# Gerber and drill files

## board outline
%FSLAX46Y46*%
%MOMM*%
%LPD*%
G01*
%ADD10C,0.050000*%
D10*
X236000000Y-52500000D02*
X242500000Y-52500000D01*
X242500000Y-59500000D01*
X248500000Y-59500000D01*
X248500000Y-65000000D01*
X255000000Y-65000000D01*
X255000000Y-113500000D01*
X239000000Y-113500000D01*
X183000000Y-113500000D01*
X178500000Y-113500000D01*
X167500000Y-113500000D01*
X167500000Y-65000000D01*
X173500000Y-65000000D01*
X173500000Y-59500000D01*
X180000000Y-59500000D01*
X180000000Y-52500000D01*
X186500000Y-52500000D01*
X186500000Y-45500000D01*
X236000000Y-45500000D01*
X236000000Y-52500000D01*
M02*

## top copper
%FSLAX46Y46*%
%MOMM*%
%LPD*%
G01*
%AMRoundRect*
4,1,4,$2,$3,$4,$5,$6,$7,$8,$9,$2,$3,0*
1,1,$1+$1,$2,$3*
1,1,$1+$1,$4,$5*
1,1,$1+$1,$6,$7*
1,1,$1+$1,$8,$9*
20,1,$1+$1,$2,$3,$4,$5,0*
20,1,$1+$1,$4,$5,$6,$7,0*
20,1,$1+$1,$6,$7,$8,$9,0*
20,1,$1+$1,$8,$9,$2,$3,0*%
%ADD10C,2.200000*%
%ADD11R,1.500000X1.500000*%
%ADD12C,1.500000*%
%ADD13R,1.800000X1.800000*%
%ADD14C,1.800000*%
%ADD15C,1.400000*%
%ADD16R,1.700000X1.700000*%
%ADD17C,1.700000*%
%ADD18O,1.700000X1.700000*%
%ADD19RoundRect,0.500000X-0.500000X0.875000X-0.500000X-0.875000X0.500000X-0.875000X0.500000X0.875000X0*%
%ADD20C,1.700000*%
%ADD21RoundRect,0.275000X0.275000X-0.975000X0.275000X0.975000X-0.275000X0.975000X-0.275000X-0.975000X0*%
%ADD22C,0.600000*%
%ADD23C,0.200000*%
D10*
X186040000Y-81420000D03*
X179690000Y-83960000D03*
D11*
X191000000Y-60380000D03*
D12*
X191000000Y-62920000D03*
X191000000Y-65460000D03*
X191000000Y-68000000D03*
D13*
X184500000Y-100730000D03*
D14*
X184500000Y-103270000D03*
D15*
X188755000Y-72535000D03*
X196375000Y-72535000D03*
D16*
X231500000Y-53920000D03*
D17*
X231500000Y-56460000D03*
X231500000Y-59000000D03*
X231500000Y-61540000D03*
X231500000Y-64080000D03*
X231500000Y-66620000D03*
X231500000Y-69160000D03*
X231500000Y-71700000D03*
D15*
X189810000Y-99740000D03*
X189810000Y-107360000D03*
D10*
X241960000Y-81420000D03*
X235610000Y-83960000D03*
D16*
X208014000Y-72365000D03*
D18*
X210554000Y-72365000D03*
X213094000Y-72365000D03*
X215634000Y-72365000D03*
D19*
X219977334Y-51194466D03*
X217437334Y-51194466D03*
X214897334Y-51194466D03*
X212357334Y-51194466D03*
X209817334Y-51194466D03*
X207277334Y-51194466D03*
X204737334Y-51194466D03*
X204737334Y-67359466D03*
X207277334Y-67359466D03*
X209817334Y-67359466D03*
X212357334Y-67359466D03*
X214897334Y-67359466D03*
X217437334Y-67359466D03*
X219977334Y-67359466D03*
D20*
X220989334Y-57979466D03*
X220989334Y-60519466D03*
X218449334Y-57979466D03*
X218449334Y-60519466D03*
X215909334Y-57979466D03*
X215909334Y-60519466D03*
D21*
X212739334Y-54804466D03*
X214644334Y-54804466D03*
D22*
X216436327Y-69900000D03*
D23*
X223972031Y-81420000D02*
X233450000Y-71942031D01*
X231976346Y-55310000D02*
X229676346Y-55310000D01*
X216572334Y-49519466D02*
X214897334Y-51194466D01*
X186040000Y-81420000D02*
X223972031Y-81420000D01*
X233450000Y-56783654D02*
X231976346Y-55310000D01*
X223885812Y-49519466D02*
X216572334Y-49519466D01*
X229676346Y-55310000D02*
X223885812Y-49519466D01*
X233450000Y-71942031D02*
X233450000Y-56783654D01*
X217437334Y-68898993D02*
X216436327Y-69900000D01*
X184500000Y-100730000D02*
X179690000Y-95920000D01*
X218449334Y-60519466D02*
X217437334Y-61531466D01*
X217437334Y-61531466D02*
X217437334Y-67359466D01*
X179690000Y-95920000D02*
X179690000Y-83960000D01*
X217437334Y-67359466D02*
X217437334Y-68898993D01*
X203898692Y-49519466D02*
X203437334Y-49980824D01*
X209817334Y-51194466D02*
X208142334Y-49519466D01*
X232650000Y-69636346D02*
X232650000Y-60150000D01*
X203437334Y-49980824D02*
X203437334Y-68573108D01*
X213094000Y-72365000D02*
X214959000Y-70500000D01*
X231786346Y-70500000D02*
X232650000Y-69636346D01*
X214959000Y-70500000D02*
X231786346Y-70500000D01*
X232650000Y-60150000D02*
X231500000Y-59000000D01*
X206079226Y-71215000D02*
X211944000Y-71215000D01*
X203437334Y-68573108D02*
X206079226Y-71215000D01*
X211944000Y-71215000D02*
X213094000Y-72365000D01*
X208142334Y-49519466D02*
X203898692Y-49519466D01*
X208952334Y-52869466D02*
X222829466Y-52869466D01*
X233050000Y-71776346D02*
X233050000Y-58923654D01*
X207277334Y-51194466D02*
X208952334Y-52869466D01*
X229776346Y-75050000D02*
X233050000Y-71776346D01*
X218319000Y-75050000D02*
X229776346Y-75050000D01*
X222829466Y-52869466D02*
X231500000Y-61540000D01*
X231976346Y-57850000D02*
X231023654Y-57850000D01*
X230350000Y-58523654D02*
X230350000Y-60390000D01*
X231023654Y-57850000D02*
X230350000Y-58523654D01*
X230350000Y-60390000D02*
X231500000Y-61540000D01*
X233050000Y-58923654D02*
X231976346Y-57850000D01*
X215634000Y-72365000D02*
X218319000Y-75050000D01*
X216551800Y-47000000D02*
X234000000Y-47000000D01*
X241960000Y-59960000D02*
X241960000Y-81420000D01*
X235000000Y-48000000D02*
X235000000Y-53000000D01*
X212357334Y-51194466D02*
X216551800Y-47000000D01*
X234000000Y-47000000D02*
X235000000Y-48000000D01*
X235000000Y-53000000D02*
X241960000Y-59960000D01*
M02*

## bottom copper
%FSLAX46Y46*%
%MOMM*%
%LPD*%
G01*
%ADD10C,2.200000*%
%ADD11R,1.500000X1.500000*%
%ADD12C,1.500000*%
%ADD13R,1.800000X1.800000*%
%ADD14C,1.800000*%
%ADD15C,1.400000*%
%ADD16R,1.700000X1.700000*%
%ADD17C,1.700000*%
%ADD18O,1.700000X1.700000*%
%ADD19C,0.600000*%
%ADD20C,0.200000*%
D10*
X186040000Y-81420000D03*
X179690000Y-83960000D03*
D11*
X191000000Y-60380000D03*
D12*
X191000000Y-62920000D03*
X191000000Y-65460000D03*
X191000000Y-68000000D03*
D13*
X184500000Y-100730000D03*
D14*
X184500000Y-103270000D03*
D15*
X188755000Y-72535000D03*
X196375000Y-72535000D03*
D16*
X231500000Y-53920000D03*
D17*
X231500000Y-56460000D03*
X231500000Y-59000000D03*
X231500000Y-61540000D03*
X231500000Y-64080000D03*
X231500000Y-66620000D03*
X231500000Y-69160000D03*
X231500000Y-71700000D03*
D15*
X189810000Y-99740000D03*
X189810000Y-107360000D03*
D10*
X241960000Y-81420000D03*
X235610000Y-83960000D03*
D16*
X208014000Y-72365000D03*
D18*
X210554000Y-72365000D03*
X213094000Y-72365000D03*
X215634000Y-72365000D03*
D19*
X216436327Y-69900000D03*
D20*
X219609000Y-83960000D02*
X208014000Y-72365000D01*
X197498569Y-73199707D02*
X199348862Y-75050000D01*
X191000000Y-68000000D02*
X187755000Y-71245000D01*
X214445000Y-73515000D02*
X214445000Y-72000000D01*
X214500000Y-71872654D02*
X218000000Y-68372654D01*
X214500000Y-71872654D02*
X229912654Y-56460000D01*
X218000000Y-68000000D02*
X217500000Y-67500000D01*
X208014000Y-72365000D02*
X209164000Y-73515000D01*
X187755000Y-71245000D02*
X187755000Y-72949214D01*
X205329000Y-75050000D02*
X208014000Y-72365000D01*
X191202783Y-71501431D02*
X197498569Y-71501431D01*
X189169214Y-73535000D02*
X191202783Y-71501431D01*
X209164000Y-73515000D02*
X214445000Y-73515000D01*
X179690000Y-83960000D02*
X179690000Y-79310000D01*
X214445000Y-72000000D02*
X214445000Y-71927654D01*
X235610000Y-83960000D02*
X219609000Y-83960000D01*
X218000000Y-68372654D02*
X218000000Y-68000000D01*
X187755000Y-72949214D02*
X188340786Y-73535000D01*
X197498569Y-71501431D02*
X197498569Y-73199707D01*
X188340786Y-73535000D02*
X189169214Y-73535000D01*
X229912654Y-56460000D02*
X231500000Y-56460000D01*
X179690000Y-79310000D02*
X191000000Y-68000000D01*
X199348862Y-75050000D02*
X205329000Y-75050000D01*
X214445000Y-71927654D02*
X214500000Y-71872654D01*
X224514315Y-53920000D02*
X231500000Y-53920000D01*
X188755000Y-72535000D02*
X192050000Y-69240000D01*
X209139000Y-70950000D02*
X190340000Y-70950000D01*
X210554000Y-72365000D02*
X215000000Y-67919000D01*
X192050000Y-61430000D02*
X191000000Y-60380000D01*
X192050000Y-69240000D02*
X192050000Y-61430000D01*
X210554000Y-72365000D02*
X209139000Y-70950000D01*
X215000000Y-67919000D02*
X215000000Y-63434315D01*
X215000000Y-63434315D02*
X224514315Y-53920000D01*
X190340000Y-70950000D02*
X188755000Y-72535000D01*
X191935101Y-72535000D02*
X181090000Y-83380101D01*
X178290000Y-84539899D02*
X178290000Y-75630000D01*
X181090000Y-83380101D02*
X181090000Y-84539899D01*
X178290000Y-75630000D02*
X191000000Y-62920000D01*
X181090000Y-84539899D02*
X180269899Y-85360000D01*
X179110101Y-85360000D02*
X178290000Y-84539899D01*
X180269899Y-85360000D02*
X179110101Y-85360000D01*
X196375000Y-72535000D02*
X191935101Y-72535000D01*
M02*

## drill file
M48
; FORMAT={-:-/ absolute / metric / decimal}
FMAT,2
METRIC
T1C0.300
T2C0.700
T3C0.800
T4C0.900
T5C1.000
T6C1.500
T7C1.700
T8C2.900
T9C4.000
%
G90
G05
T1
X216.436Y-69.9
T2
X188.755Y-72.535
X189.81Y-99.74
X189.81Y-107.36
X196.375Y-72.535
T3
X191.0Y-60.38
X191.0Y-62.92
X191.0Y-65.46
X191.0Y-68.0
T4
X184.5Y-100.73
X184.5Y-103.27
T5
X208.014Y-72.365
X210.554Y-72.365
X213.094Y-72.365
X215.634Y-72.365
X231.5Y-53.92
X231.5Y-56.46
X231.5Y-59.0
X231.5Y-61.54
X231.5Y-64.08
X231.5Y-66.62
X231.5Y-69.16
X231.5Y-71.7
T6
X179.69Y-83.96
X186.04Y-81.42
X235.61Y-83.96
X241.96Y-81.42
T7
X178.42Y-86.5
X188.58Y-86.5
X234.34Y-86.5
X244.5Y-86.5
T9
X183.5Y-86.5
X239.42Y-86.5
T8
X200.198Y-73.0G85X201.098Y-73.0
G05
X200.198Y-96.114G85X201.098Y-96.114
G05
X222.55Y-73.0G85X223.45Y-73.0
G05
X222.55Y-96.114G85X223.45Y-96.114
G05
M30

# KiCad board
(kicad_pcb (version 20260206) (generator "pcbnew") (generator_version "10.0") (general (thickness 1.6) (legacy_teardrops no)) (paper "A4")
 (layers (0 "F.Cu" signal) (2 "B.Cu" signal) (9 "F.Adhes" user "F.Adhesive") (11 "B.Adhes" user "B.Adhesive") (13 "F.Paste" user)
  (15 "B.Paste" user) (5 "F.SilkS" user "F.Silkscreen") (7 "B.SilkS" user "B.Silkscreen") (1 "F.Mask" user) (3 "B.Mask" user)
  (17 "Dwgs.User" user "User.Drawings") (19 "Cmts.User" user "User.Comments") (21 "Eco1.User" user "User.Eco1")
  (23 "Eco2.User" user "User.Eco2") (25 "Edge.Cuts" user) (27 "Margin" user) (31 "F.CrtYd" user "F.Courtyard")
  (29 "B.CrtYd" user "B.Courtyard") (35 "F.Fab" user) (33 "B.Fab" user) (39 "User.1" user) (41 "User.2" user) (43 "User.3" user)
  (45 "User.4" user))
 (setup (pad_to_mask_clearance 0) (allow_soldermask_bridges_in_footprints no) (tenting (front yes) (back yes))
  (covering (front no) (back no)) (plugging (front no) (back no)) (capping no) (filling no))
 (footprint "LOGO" (layer "F.Cu") (at 224.5 107)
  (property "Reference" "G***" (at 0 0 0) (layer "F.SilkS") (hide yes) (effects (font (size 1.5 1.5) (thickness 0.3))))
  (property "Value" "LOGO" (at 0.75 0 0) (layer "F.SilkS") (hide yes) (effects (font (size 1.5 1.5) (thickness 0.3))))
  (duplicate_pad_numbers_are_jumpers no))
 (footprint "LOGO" (layer "F.Cu") (at 238 54)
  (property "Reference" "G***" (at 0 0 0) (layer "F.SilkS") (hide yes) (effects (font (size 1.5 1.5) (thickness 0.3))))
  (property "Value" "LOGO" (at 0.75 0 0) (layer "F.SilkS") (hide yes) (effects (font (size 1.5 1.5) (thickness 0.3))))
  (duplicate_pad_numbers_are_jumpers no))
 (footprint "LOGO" (layer "F.Cu") (at 202.605439 106.48253)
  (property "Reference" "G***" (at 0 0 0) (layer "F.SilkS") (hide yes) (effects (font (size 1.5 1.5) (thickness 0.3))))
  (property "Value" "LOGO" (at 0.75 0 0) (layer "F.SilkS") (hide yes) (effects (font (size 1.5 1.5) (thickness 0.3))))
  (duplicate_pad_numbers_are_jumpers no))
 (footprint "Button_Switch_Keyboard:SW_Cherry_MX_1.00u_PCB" (layer "F.Cu") (at 186.04 81.42)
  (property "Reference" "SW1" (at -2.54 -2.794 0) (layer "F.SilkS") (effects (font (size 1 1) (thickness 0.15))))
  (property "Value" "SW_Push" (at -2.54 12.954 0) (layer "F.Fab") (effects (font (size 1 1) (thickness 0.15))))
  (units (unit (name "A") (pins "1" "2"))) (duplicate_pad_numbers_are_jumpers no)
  (pad "" np_thru_hole circle (at -7.62 5.08) (size 1.7 1.7) (drill 1.7) (layers "*.Cu" "*.Mask"))
  (pad "" np_thru_hole circle (at -2.54 5.08) (size 4 4) (drill 4) (layers "*.Cu" "*.Mask"))
  (pad "" np_thru_hole circle (at 2.54 5.08) (size 1.7 1.7) (drill 1.7) (layers "*.Cu" "*.Mask"))
  (pad "1" thru_hole circle (at 0 0) (size 2.2 2.2) (drill 1.5) (layers "*.Cu" "*.Mask") (remove_unused_layers no) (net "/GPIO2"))
  (pad "2" thru_hole circle (at -6.35 2.54) (size 2.2 2.2) (drill 1.5) (layers "*.Cu" "*.Mask") (remove_unused_layers no) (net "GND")))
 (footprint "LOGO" (layer "F.Cu") (at 172.5 71.5)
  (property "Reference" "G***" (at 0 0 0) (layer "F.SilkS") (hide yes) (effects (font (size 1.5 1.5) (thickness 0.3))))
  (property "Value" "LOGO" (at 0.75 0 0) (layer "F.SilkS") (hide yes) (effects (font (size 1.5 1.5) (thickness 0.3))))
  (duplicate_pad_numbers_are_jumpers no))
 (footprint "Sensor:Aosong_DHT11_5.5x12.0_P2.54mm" (layer "F.Cu") (at 191 60.38)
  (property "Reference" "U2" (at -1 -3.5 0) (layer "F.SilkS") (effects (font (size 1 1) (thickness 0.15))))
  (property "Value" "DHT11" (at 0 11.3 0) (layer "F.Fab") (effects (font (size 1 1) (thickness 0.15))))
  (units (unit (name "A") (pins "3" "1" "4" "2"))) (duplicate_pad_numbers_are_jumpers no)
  (pad "1" thru_hole rect (at 0 0) (size 1.5 1.5) (drill 0.8) (layers "*.Cu" "*.Mask") (remove_unused_layers no) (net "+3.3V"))
  (pad "2" thru_hole circle (at 0 2.54) (size 1.5 1.5) (drill 0.8) (layers "*.Cu" "*.Mask") (remove_unused_layers no) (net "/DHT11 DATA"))
  (pad "3" thru_hole circle (at 0 5.08) (size 1.5 1.5) (drill 0.8) (layers "*.Cu" "*.Mask") (remove_unused_layers no)
   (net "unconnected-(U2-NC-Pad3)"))
  (pad "4" thru_hole circle (at 0 7.62) (size 1.5 1.5) (drill 0.8) (layers "*.Cu" "*.Mask") (remove_unused_layers no) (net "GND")))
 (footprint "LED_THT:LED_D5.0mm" (layer "F.Cu") (at 184.5 100.73 -90)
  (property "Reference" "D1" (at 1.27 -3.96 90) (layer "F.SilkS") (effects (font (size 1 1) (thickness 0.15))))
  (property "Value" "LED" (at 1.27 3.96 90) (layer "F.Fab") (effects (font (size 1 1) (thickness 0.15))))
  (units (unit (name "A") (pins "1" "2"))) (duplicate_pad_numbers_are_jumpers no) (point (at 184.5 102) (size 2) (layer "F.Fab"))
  (pad "1" thru_hole rect (at 0 0 270) (size 1.8 1.8) (drill 0.9) (layers "*.Cu" "*.Mask") (remove_unused_layers no) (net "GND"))
  (pad "2" thru_hole circle (at 2.54 0 270) (size 1.8 1.8) (drill 0.9) (layers "*.Cu" "*.Mask") (remove_unused_layers no)))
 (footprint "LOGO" (layer "F.Cu") (at 248.5 70)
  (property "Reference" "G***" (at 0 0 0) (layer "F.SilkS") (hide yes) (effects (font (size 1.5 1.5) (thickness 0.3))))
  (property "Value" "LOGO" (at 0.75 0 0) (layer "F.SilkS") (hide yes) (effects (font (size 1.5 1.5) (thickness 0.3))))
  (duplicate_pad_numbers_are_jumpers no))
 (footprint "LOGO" (layer "F.Cu") (at 194 51)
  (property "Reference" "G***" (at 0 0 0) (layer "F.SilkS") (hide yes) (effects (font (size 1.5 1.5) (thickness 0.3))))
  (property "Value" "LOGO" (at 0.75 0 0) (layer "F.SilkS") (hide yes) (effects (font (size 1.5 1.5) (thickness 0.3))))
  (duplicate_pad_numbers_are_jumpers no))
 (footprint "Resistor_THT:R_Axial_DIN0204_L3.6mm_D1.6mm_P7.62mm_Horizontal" (layer "F.Cu") (at 188.755 72.535)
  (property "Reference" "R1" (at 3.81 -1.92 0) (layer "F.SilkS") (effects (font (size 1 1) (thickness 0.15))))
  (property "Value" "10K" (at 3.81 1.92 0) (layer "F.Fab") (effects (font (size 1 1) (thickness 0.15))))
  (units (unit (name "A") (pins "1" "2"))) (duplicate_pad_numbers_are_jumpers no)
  (pad "1" thru_hole circle (at 0 0) (size 1.4 1.4) (drill 0.7) (layers "*.Cu" "*.Mask") (remove_unused_layers no) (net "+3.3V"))
  (pad "2" thru_hole circle (at 7.62 0) (size 1.4 1.4) (drill 0.7) (layers "*.Cu" "*.Mask") (remove_unused_layers no) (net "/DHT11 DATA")))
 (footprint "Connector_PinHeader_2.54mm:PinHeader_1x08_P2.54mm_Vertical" (layer "F.Cu") (at 231.5 53.92)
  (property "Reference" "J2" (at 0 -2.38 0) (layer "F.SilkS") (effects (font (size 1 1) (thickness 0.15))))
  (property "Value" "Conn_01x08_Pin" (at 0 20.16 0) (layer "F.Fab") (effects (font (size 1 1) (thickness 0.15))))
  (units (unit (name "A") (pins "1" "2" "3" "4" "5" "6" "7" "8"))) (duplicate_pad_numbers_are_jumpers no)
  (pad "1" thru_hole rect (at 0 0) (size 1.7 1.7) (drill 1) (layers "*.Cu" "*.Mask") (remove_unused_layers no) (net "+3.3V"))
  (pad "2" thru_hole circle (at 0 2.54) (size 1.7 1.7) (drill 1) (layers "*.Cu" "*.Mask") (remove_unused_layers no) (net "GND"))
  (pad "3" thru_hole circle (at 0 5.08) (size 1.7 1.7) (drill 1) (layers "*.Cu" "*.Mask") (remove_unused_layers no) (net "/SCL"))
  (pad "4" thru_hole circle (at 0 7.62) (size 1.7 1.7) (drill 1) (layers "*.Cu" "*.Mask") (remove_unused_layers no) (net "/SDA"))
  (pad "5" thru_hole circle (at 0 10.16) (size 1.7 1.7) (drill 1) (layers "*.Cu" "*.Mask") (remove_unused_layers no)
   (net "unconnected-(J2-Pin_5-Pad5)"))
  (pad "6" thru_hole circle (at 0 12.7) (size 1.7 1.7) (drill 1) (layers "*.Cu" "*.Mask") (remove_unused_layers no)
   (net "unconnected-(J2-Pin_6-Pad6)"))
  (pad "7" thru_hole circle (at 0 15.24) (size 1.7 1.7) (drill 1) (layers "*.Cu" "*.Mask") (remove_unused_layers no)
   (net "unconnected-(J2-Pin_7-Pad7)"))
  (pad "8" thru_hole circle (at 0 17.78) (size 1.7 1.7) (drill 1) (layers "*.Cu" "*.Mask") (remove_unused_layers no)
   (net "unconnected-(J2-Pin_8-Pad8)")))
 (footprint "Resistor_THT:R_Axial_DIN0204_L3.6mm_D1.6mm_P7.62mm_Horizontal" (layer "F.Cu") (at 189.81 99.74 -90)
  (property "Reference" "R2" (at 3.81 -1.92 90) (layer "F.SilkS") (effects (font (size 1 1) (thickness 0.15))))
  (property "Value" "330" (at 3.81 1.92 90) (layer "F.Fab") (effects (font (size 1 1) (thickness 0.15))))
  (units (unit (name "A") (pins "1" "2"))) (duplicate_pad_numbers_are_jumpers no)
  (pad "1" thru_hole circle (at 0 0 270) (size 1.4 1.4) (drill 0.7) (layers "*.Cu" "*.Mask") (remove_unused_layers no) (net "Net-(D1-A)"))
  (pad "2" thru_hole circle (at 7.62 0 270) (size 1.4 1.4) (drill 0.7) (layers "*.Cu" "*.Mask") (remove_unused_layers no)))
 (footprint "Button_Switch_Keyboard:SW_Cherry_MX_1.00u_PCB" (layer "F.Cu") (at 241.96 81.42)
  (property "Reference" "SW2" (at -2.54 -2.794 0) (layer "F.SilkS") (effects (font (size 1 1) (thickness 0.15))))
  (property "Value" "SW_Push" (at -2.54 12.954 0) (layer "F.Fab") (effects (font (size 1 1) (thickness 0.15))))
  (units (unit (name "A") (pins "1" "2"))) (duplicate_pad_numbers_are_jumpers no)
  (pad "" np_thru_hole circle (at -7.62 5.08) (size 1.7 1.7) (drill 1.7) (layers "*.Cu" "*.Mask"))
  (pad "" np_thru_hole circle (at -2.54 5.08) (size 4 4) (drill 4) (layers "*.Cu" "*.Mask"))
  (pad "" np_thru_hole circle (at 2.54 5.08) (size 1.7 1.7) (drill 1.7) (layers "*.Cu" "*.Mask"))
  (pad "1" thru_hole circle (at 0 0) (size 2.2 2.2) (drill 1.5) (layers "*.Cu" "*.Mask") (remove_unused_layers no) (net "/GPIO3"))
  (pad "2" thru_hole circle (at -6.35 2.54) (size 2.2 2.2) (drill 1.5) (layers "*.Cu" "*.Mask") (remove_unused_layers no) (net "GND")))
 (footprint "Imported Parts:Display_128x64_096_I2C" (layer "F.Cu") (at 211.824 72.365)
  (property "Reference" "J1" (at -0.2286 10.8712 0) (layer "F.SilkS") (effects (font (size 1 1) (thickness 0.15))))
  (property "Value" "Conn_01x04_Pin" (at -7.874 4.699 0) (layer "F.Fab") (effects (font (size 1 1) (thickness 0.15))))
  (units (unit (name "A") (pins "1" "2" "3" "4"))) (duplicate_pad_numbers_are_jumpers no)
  (pad "" np_thru_hole oval (at -11.176 0.635) (size 3.8 2.9) (drill oval 3.8 2.9) (layers "*.Cu" "*.Mask"))
  (pad "" np_thru_hole oval (at -11.176 23.749) (size 3.8 2.9) (drill oval 3.8 2.9) (layers "*.Cu" "*.Mask"))
  (pad "" np_thru_hole oval (at 11.176 0.635) (size 3.8 2.9) (drill oval 3.8 2.9) (layers "*.Cu" "*.Mask"))
  (pad "" np_thru_hole oval (at 11.176 23.749) (size 3.8 2.9) (drill oval 3.8 2.9) (layers "*.Cu" "*.Mask"))
  (pad "1" thru_hole rect (at -3.81 0 90) (size 1.7 1.7) (drill 1) (layers "*.Cu" "*.Mask") (remove_unused_layers no) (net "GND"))
  (pad "2" thru_hole oval (at -1.27 0 90) (size 1.7 1.7) (drill 1) (layers "*.Cu" "*.Mask") (remove_unused_layers no) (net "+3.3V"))
  (pad "3" thru_hole oval (at 1.27 0 90) (size 1.7 1.7) (drill 1) (layers "*.Cu" "*.Mask") (remove_unused_layers no) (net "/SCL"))
  (pad "4" thru_hole oval (at 3.81 0 90) (size 1.7 1.7) (drill 1) (layers "*.Cu" "*.Mask") (remove_unused_layers no) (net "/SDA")))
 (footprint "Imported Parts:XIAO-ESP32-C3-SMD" (layer "F.Cu") (at 201.857334 50.359466 -90)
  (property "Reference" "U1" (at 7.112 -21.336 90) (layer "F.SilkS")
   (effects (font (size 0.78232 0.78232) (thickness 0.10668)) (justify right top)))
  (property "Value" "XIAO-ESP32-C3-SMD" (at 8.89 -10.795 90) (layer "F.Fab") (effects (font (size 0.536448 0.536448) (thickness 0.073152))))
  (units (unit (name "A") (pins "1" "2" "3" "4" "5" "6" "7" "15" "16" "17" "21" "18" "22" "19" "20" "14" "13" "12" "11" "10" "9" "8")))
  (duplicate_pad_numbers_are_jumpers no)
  (pad "1" smd roundrect (at 0.835 -18.12 270) (size 2.75 2) (layers "F.Cu" "F.Mask" "F.Paste") (roundrect_rratio 0.25)
   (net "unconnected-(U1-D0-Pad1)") (solder_mask_margin 0.0508) (thermal_bridge_angle 45))
  (pad "2" smd roundrect (at 0.835 -15.58 270) (size 2.75 2) (layers "F.Cu" "F.Mask" "F.Paste") (roundrect_rratio 0.25) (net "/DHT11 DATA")
   (solder_mask_margin 0.0508) (thermal_bridge_angle 45))
  (pad "3" smd roundrect (at 0.835 -13.04 270) (size 2.75 2) (layers "F.Cu" "F.Mask" "F.Paste") (roundrect_rratio 0.25) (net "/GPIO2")
   (solder_mask_margin 0.0508) (thermal_bridge_angle 45))
  (pad "4" smd roundrect (at 0.835 -10.5 270) (size 2.75 2) (layers "F.Cu" "F.Mask" "F.Paste") (roundrect_rratio 0.25) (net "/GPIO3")
   (solder_mask_margin 0.0508) (thermal_bridge_angle 45))
  (pad "5" smd roundrect (at 0.835 -7.96 270) (size 2.75 2) (layers "F.Cu" "F.Mask" "F.Paste") (roundrect_rratio 0.25) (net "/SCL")
   (solder_mask_margin 0.0508) (thermal_bridge_angle 45))
  (pad "6" smd roundrect (at 0.835 -5.42 270) (size 2.75 2) (layers "F.Cu" "F.Mask" "F.Paste") (roundrect_rratio 0.25) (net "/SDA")
   (solder_mask_margin 0.0508) (thermal_bridge_angle 45))
  (pad "7" smd roundrect (at 0.835 -2.88 270) (size 2.75 2) (layers "F.Cu" "F.Mask" "F.Paste") (roundrect_rratio 0.25) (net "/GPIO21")
   (solder_mask_margin 0.0508) (thermal_bridge_angle 45))
  (pad "8" smd roundrect (at 17 -2.88 270) (size 2.75 2) (layers "F.Cu" "F.Mask" "F.Paste") (roundrect_rratio 0.25)
   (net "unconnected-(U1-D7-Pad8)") (solder_mask_margin 0.0508) (thermal_bridge_angle 45))
  (pad "9" smd roundrect (at 17 -5.42 270) (size 2.75 2) (layers "F.Cu" "F.Mask" "F.Paste") (roundrect_rratio 0.25)
   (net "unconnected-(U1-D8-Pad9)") (solder_mask_margin 0.0508) (thermal_bridge_angle 45))
  (pad "10" smd roundrect (at 17 -7.96 270) (size 2.75 2) (layers "F.Cu" "F.Mask" "F.Paste") (roundrect_rratio 0.25)
   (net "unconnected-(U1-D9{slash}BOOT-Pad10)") (solder_mask_margin 0.0508) (thermal_bridge_angle 45))
  (pad "11" smd roundrect (at 17 -10.5 270) (size 2.75 2) (layers "F.Cu" "F.Mask" "F.Paste") (roundrect_rratio 0.25)
   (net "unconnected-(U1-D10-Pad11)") (solder_mask_margin 0.0508) (thermal_bridge_angle 45))
  (pad "12" smd roundrect (at 17 -13.04 270) (size 2.75 2) (layers "F.Cu" "F.Mask" "F.Paste") (roundrect_rratio 0.25) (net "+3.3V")
   (solder_mask_margin 0.0508) (thermal_bridge_angle 45))
  (pad "13" smd roundrect (at 17 -15.58 270) (size 2.75 2) (layers "F.Cu" "F.Mask" "F.Paste") (roundrect_rratio 0.25) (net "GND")
   (solder_mask_margin 0.0508) (thermal_bridge_angle 45))
  (pad "14" smd roundrect (at 17 -18.12 270) (size 2.75 2) (layers "F.Cu" "F.Mask" "F.Paste") (roundrect_rratio 0.25) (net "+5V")
   (solder_mask_margin 0.0508) (thermal_bridge_angle 45))
  (pad "15" smd circle (at 7.62 -19.132 270) (size 1.7 1.7) (layers "F.Cu" "F.Mask" "F.Paste") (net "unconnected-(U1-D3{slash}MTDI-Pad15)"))
  (pad "16" smd circle (at 10.16 -19.132 270) (size 1.7 1.7) (layers "F.Cu" "F.Mask" "F.Paste") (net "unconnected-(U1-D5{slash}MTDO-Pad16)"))
  (pad "17" smd circle (at 7.62 -16.592 270) (size 1.7 1.7) (layers "F.Cu" "F.Mask" "F.Paste") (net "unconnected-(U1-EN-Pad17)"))
  (pad "18" smd circle (at 10.16 -16.592 270) (size 1.7 1.7) (layers "F.Cu" "F.Mask" "F.Paste") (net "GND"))
  (pad "19" smd circle (at 7.62 -14.052 270) (size 1.7 1.7) (layers "F.Cu" "F.Mask" "F.Paste") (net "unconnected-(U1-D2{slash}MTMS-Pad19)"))
  (pad "20" smd circle (at 10.16 -14.052 270) (size 1.7 1.7) (layers "F.Cu" "F.Mask" "F.Paste") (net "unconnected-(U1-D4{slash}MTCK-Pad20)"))
  (pad "21" smd roundrect (at 4.445 -10.882 90) (size 2.5 1.1) (layers "F.Cu" "F.Mask" "F.Paste") (roundrect_rratio 0.25)
   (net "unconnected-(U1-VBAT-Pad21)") (thermal_bridge_angle 45))
  (pad "22" smd roundrect (at 4.445 -12.787 90) (size 2.5 1.1) (layers "F.Cu" "F.Mask" "F.Paste") (roundrect_rratio 0.25)
   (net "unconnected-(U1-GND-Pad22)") (thermal_bridge_angle 45)))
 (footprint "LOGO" (layer "F.Cu") (at 246.5 104.5)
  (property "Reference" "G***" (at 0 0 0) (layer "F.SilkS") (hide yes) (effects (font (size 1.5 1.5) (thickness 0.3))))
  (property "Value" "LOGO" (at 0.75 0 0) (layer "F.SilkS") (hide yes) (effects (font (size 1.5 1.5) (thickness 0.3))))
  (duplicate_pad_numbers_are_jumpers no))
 (gr_poly
  (pts (xy 236 52.5) (xy 242.5 52.5) (xy 242.5 59.5) (xy 248.5 59.5) (xy 248.5 65) (xy 255 65) (xy 255 113.5) (xy 239 113.5) (xy 183 113.5)
   (xy 178.5 113.5) (xy 167.5 113.5) (xy 167.5 65) (xy 173.5 65) (xy 173.5 59.5) (xy 180 59.5) (xy 180 52.5) (xy 186.5 52.5) (xy 186.5 45.5)
   (xy 236 45.5))
  (stroke (width 0.05) (type default)) (fill no) (layer "Edge.Cuts"))
 (segment (start 223.972031 81.42) (end 233.45 71.942031) (width 0.2) (layer "F.Cu") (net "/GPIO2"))
 (segment (start 231.976346 55.31) (end 229.676346 55.31) (width 0.2) (layer "F.Cu") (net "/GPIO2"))
 (segment (start 216.572334 49.519466) (end 214.897334 51.194466) (width 0.2) (layer "F.Cu") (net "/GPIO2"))
 (segment (start 186.04 81.42) (end 223.972031 81.42) (width 0.2) (layer "F.Cu") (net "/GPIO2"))
 (segment (start 233.45 56.783654) (end 231.976346 55.31) (width 0.2) (layer "F.Cu") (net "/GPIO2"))
 (segment (start 223.885812 49.519466) (end 216.572334 49.519466) (width 0.2) (layer "F.Cu") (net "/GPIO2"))
 (segment (start 229.676346 55.31) (end 223.885812 49.519466) (width 0.2) (layer "F.Cu") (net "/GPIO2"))
 (segment (start 233.45 71.942031) (end 233.45 56.783654) (width 0.2) (layer "F.Cu") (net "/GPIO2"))
 (segment (start 217.437334 68.898993) (end 216.436327 69.9) (width 0.2) (layer "F.Cu") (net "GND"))
 (segment (start 184.5 100.73) (end 179.69 95.92) (width 0.2) (layer "F.Cu") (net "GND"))
 (segment (start 218.449334 60.519466) (end 217.437334 61.531466) (width 0.2) (layer "F.Cu") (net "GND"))
 (segment (start 217.437334 61.531466) (end 217.437334 67.359466) (width 0.2) (layer "F.Cu") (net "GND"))
 (segment (start 179.69 95.92) (end 179.69 83.96) (width 0.2) (layer "F.Cu") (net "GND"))
 (segment (start 217.437334 67.359466) (end 217.437334 68.898993) (width 0.2) (layer "F.Cu") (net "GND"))
 (via (at 216.436327 69.9) (size 0.6) (drill 0.3) (layers "F.Cu" "B.Cu") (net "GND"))
 (segment (start 219.609 83.96) (end 208.014 72.365) (width 0.2) (layer "B.Cu") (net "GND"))
 (segment (start 197.498569 73.199707) (end 199.348862 75.05) (width 0.2) (layer "B.Cu") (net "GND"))
 (segment (start 191 68) (end 187.755 71.245) (width 0.2) (layer "B.Cu") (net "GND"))
 (segment (start 214.445 73.515) (end 214.445 72) (width 0.2) (layer "B.Cu") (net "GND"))
 (segment (start 214.5 71.872654) (end 218 68.372654) (width 0.2) (layer "B.Cu") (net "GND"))
 (segment (start 214.5 71.872654) (end 229.912654 56.46) (width 0.2) (layer "B.Cu") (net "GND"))
 (segment (start 218 68) (end 217.5 67.5) (width 0.2) (layer "B.Cu") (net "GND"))
 (segment (start 208.014 72.365) (end 209.164 73.515) (width 0.2) (layer "B.Cu") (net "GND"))
 (segment (start 187.755 71.245) (end 187.755 72.949214) (width 0.2) (layer "B.Cu") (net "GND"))
 (segment (start 205.329 75.05) (end 208.014 72.365) (width 0.2) (layer "B.Cu") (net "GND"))
 (segment (start 191.202783 71.501431) (end 197.498569 71.501431) (width 0.2) (layer "B.Cu") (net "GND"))
 (segment (start 189.169214 73.535) (end 191.202783 71.501431) (width 0.2) (layer "B.Cu") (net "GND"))
 (segment (start 209.164 73.515) (end 214.445 73.515) (width 0.2) (layer "B.Cu") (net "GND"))
 (segment (start 179.69 83.96) (end 179.69 79.31) (width 0.2) (layer "B.Cu") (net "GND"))
 (segment (start 214.445 72) (end 214.445 71.927654) (width 0.2) (layer "B.Cu") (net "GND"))
 (segment (start 235.61 83.96) (end 219.609 83.96) (width 0.2) (layer "B.Cu") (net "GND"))
 (segment (start 218 68.372654) (end 218 68) (width 0.2) (layer "B.Cu") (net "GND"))
 (segment (start 187.755 72.949214) (end 188.340786 73.535) (width 0.2) (layer "B.Cu") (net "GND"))
 (segment (start 197.498569 71.501431) (end 197.498569 73.199707) (width 0.2) (layer "B.Cu") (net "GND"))
 (segment (start 188.340786 73.535) (end 189.169214 73.535) (width 0.2) (layer "B.Cu") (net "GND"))
 (segment (start 229.912654 56.46) (end 231.5 56.46) (width 0.2) (layer "B.Cu") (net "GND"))
 (segment (start 179.69 79.31) (end 191 68) (width 0.2) (layer "B.Cu") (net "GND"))
 (segment (start 199.348862 75.05) (end 205.329 75.05) (width 0.2) (layer "B.Cu") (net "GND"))
 (segment (start 214.445 71.927654) (end 214.5 71.872654) (width 0.2) (layer "B.Cu") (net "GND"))
 (segment (start 224.514315 53.92) (end 231.5 53.92) (width 0.2) (layer "B.Cu") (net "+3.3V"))
 (segment (start 188.755 72.535) (end 192.05 69.24) (width 0.2) (layer "B.Cu") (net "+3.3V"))
 (segment (start 209.139 70.95) (end 190.34 70.95) (width 0.2) (layer "B.Cu") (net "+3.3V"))
 (segment (start 210.554 72.365) (end 215 67.919) (width 0.2) (layer "B.Cu") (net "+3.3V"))
 (segment (start 192.05 61.43) (end 191 60.38) (width 0.2) (layer "B.Cu") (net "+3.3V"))
 (segment (start 192.05 69.24) (end 192.05 61.43) (width 0.2) (layer "B.Cu") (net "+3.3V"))
 (segment (start 210.554 72.365) (end 209.139 70.95) (width 0.2) (layer "B.Cu") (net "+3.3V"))
 (segment (start 215 67.919) (end 215 63.434315) (width 0.2) (layer "B.Cu") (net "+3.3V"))
 (segment (start 215 63.434315) (end 224.514315 53.92) (width 0.2) (layer "B.Cu") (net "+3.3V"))
 (segment (start 190.34 70.95) (end 188.755 72.535) (width 0.2) (layer "B.Cu") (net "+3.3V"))
 (segment (start 191.935101 72.535) (end 181.09 83.380101) (width 0.2) (layer "B.Cu") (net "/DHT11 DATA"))
 (segment (start 178.29 84.539899) (end 178.29 75.63) (width 0.2) (layer "B.Cu") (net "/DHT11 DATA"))
 (segment (start 181.09 83.380101) (end 181.09 84.539899) (width 0.2) (layer "B.Cu") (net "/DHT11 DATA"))
 (segment (start 178.29 75.63) (end 191 62.92) (width 0.2) (layer "B.Cu") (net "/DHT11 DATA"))
 (segment (start 181.09 84.539899) (end 180.269899 85.36) (width 0.2) (layer "B.Cu") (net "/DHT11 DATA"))
 (segment (start 179.110101 85.36) (end 178.29 84.539899) (width 0.2) (layer "B.Cu") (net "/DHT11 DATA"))
 (segment (start 180.269899 85.36) (end 179.110101 85.36) (width 0.2) (layer "B.Cu") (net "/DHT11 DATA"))
 (segment (start 196.375 72.535) (end 191.935101 72.535) (width 0.2) (layer "B.Cu") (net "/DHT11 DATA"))
 (segment (start 203.898692 49.519466) (end 203.437334 49.980824) (width 0.2) (layer "F.Cu") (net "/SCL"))
 (segment (start 209.817334 51.194466) (end 208.142334 49.519466) (width 0.2) (layer "F.Cu") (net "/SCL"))
 (segment (start 232.65 69.636346) (end 232.65 60.15) (width 0.2) (layer "F.Cu") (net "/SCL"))
 (segment (start 203.437334 49.980824) (end 203.437334 68.573108) (width 0.2) (layer "F.Cu") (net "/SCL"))
 (segment (start 213.094 72.365) (end 214.959 70.5) (width 0.2) (layer "F.Cu") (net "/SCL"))
 (segment (start 231.786346 70.5) (end 232.65 69.636346) (width 0.2) (layer "F.Cu") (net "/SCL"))
 (segment (start 214.959 70.5) (end 231.786346 70.5) (width 0.2) (layer "F.Cu") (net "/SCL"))
 (segment (start 232.65 60.15) (end 231.5 59) (width 0.2) (layer "F.Cu") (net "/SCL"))
 (segment (start 206.079226 71.215) (end 211.944 71.215) (width 0.2) (layer "F.Cu") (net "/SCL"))
 (segment (start 203.437334 68.573108) (end 206.079226 71.215) (width 0.2) (layer "F.Cu") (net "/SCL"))
 (segment (start 211.944 71.215) (end 213.094 72.365) (width 0.2) (layer "F.Cu") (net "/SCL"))
 (segment (start 208.142334 49.519466) (end 203.898692 49.519466) (width 0.2) (layer "F.Cu") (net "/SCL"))
 (segment (start 208.952334 52.869466) (end 222.829466 52.869466) (width 0.2) (layer "F.Cu") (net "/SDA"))
 (segment (start 233.05 71.776346) (end 233.05 58.923654) (width 0.2) (layer "F.Cu") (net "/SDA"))
 (segment (start 207.277334 51.194466) (end 208.952334 52.869466) (width 0.2) (layer "F.Cu") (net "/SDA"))
 (segment (start 229.776346 75.05) (end 233.05 71.776346) (width 0.2) (layer "F.Cu") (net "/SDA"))
 (segment (start 218.319 75.05) (end 229.776346 75.05) (width 0.2) (layer "F.Cu") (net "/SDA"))
 (segment (start 222.829466 52.869466) (end 231.5 61.54) (width 0.2) (layer "F.Cu") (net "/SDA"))
 (segment (start 231.976346 57.85) (end 231.023654 57.85) (width 0.2) (layer "F.Cu") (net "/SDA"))
 (segment (start 230.35 58.523654) (end 230.35 60.39) (width 0.2) (layer "F.Cu") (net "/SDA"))
 (segment (start 231.023654 57.85) (end 230.35 58.523654) (width 0.2) (layer "F.Cu") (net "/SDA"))
 (segment (start 230.35 60.39) (end 231.5 61.54) (width 0.2) (layer "F.Cu") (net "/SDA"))
 (segment (start 233.05 58.923654) (end 231.976346 57.85) (width 0.2) (layer "F.Cu") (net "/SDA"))
 (segment (start 215.634 72.365) (end 218.319 75.05) (width 0.2) (layer "F.Cu") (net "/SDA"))
 (segment (start 216.5518 47) (end 234 47) (width 0.2) (layer "F.Cu") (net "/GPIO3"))
 (segment (start 241.96 59.96) (end 241.96 81.42) (width 0.2) (layer "F.Cu") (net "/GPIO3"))
 (segment (start 235 48) (end 235 53) (width 0.2) (layer "F.Cu") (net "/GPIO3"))
 (segment (start 212.357334 51.194466) (end 216.5518 47) (width 0.2) (layer "F.Cu") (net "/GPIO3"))
 (segment (start 234 47) (end 235 48) (width 0.2) (layer "F.Cu") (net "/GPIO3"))
 (segment (start 235 53) (end 241.96 59.96) (width 0.2) (layer "F.Cu") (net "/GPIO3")))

